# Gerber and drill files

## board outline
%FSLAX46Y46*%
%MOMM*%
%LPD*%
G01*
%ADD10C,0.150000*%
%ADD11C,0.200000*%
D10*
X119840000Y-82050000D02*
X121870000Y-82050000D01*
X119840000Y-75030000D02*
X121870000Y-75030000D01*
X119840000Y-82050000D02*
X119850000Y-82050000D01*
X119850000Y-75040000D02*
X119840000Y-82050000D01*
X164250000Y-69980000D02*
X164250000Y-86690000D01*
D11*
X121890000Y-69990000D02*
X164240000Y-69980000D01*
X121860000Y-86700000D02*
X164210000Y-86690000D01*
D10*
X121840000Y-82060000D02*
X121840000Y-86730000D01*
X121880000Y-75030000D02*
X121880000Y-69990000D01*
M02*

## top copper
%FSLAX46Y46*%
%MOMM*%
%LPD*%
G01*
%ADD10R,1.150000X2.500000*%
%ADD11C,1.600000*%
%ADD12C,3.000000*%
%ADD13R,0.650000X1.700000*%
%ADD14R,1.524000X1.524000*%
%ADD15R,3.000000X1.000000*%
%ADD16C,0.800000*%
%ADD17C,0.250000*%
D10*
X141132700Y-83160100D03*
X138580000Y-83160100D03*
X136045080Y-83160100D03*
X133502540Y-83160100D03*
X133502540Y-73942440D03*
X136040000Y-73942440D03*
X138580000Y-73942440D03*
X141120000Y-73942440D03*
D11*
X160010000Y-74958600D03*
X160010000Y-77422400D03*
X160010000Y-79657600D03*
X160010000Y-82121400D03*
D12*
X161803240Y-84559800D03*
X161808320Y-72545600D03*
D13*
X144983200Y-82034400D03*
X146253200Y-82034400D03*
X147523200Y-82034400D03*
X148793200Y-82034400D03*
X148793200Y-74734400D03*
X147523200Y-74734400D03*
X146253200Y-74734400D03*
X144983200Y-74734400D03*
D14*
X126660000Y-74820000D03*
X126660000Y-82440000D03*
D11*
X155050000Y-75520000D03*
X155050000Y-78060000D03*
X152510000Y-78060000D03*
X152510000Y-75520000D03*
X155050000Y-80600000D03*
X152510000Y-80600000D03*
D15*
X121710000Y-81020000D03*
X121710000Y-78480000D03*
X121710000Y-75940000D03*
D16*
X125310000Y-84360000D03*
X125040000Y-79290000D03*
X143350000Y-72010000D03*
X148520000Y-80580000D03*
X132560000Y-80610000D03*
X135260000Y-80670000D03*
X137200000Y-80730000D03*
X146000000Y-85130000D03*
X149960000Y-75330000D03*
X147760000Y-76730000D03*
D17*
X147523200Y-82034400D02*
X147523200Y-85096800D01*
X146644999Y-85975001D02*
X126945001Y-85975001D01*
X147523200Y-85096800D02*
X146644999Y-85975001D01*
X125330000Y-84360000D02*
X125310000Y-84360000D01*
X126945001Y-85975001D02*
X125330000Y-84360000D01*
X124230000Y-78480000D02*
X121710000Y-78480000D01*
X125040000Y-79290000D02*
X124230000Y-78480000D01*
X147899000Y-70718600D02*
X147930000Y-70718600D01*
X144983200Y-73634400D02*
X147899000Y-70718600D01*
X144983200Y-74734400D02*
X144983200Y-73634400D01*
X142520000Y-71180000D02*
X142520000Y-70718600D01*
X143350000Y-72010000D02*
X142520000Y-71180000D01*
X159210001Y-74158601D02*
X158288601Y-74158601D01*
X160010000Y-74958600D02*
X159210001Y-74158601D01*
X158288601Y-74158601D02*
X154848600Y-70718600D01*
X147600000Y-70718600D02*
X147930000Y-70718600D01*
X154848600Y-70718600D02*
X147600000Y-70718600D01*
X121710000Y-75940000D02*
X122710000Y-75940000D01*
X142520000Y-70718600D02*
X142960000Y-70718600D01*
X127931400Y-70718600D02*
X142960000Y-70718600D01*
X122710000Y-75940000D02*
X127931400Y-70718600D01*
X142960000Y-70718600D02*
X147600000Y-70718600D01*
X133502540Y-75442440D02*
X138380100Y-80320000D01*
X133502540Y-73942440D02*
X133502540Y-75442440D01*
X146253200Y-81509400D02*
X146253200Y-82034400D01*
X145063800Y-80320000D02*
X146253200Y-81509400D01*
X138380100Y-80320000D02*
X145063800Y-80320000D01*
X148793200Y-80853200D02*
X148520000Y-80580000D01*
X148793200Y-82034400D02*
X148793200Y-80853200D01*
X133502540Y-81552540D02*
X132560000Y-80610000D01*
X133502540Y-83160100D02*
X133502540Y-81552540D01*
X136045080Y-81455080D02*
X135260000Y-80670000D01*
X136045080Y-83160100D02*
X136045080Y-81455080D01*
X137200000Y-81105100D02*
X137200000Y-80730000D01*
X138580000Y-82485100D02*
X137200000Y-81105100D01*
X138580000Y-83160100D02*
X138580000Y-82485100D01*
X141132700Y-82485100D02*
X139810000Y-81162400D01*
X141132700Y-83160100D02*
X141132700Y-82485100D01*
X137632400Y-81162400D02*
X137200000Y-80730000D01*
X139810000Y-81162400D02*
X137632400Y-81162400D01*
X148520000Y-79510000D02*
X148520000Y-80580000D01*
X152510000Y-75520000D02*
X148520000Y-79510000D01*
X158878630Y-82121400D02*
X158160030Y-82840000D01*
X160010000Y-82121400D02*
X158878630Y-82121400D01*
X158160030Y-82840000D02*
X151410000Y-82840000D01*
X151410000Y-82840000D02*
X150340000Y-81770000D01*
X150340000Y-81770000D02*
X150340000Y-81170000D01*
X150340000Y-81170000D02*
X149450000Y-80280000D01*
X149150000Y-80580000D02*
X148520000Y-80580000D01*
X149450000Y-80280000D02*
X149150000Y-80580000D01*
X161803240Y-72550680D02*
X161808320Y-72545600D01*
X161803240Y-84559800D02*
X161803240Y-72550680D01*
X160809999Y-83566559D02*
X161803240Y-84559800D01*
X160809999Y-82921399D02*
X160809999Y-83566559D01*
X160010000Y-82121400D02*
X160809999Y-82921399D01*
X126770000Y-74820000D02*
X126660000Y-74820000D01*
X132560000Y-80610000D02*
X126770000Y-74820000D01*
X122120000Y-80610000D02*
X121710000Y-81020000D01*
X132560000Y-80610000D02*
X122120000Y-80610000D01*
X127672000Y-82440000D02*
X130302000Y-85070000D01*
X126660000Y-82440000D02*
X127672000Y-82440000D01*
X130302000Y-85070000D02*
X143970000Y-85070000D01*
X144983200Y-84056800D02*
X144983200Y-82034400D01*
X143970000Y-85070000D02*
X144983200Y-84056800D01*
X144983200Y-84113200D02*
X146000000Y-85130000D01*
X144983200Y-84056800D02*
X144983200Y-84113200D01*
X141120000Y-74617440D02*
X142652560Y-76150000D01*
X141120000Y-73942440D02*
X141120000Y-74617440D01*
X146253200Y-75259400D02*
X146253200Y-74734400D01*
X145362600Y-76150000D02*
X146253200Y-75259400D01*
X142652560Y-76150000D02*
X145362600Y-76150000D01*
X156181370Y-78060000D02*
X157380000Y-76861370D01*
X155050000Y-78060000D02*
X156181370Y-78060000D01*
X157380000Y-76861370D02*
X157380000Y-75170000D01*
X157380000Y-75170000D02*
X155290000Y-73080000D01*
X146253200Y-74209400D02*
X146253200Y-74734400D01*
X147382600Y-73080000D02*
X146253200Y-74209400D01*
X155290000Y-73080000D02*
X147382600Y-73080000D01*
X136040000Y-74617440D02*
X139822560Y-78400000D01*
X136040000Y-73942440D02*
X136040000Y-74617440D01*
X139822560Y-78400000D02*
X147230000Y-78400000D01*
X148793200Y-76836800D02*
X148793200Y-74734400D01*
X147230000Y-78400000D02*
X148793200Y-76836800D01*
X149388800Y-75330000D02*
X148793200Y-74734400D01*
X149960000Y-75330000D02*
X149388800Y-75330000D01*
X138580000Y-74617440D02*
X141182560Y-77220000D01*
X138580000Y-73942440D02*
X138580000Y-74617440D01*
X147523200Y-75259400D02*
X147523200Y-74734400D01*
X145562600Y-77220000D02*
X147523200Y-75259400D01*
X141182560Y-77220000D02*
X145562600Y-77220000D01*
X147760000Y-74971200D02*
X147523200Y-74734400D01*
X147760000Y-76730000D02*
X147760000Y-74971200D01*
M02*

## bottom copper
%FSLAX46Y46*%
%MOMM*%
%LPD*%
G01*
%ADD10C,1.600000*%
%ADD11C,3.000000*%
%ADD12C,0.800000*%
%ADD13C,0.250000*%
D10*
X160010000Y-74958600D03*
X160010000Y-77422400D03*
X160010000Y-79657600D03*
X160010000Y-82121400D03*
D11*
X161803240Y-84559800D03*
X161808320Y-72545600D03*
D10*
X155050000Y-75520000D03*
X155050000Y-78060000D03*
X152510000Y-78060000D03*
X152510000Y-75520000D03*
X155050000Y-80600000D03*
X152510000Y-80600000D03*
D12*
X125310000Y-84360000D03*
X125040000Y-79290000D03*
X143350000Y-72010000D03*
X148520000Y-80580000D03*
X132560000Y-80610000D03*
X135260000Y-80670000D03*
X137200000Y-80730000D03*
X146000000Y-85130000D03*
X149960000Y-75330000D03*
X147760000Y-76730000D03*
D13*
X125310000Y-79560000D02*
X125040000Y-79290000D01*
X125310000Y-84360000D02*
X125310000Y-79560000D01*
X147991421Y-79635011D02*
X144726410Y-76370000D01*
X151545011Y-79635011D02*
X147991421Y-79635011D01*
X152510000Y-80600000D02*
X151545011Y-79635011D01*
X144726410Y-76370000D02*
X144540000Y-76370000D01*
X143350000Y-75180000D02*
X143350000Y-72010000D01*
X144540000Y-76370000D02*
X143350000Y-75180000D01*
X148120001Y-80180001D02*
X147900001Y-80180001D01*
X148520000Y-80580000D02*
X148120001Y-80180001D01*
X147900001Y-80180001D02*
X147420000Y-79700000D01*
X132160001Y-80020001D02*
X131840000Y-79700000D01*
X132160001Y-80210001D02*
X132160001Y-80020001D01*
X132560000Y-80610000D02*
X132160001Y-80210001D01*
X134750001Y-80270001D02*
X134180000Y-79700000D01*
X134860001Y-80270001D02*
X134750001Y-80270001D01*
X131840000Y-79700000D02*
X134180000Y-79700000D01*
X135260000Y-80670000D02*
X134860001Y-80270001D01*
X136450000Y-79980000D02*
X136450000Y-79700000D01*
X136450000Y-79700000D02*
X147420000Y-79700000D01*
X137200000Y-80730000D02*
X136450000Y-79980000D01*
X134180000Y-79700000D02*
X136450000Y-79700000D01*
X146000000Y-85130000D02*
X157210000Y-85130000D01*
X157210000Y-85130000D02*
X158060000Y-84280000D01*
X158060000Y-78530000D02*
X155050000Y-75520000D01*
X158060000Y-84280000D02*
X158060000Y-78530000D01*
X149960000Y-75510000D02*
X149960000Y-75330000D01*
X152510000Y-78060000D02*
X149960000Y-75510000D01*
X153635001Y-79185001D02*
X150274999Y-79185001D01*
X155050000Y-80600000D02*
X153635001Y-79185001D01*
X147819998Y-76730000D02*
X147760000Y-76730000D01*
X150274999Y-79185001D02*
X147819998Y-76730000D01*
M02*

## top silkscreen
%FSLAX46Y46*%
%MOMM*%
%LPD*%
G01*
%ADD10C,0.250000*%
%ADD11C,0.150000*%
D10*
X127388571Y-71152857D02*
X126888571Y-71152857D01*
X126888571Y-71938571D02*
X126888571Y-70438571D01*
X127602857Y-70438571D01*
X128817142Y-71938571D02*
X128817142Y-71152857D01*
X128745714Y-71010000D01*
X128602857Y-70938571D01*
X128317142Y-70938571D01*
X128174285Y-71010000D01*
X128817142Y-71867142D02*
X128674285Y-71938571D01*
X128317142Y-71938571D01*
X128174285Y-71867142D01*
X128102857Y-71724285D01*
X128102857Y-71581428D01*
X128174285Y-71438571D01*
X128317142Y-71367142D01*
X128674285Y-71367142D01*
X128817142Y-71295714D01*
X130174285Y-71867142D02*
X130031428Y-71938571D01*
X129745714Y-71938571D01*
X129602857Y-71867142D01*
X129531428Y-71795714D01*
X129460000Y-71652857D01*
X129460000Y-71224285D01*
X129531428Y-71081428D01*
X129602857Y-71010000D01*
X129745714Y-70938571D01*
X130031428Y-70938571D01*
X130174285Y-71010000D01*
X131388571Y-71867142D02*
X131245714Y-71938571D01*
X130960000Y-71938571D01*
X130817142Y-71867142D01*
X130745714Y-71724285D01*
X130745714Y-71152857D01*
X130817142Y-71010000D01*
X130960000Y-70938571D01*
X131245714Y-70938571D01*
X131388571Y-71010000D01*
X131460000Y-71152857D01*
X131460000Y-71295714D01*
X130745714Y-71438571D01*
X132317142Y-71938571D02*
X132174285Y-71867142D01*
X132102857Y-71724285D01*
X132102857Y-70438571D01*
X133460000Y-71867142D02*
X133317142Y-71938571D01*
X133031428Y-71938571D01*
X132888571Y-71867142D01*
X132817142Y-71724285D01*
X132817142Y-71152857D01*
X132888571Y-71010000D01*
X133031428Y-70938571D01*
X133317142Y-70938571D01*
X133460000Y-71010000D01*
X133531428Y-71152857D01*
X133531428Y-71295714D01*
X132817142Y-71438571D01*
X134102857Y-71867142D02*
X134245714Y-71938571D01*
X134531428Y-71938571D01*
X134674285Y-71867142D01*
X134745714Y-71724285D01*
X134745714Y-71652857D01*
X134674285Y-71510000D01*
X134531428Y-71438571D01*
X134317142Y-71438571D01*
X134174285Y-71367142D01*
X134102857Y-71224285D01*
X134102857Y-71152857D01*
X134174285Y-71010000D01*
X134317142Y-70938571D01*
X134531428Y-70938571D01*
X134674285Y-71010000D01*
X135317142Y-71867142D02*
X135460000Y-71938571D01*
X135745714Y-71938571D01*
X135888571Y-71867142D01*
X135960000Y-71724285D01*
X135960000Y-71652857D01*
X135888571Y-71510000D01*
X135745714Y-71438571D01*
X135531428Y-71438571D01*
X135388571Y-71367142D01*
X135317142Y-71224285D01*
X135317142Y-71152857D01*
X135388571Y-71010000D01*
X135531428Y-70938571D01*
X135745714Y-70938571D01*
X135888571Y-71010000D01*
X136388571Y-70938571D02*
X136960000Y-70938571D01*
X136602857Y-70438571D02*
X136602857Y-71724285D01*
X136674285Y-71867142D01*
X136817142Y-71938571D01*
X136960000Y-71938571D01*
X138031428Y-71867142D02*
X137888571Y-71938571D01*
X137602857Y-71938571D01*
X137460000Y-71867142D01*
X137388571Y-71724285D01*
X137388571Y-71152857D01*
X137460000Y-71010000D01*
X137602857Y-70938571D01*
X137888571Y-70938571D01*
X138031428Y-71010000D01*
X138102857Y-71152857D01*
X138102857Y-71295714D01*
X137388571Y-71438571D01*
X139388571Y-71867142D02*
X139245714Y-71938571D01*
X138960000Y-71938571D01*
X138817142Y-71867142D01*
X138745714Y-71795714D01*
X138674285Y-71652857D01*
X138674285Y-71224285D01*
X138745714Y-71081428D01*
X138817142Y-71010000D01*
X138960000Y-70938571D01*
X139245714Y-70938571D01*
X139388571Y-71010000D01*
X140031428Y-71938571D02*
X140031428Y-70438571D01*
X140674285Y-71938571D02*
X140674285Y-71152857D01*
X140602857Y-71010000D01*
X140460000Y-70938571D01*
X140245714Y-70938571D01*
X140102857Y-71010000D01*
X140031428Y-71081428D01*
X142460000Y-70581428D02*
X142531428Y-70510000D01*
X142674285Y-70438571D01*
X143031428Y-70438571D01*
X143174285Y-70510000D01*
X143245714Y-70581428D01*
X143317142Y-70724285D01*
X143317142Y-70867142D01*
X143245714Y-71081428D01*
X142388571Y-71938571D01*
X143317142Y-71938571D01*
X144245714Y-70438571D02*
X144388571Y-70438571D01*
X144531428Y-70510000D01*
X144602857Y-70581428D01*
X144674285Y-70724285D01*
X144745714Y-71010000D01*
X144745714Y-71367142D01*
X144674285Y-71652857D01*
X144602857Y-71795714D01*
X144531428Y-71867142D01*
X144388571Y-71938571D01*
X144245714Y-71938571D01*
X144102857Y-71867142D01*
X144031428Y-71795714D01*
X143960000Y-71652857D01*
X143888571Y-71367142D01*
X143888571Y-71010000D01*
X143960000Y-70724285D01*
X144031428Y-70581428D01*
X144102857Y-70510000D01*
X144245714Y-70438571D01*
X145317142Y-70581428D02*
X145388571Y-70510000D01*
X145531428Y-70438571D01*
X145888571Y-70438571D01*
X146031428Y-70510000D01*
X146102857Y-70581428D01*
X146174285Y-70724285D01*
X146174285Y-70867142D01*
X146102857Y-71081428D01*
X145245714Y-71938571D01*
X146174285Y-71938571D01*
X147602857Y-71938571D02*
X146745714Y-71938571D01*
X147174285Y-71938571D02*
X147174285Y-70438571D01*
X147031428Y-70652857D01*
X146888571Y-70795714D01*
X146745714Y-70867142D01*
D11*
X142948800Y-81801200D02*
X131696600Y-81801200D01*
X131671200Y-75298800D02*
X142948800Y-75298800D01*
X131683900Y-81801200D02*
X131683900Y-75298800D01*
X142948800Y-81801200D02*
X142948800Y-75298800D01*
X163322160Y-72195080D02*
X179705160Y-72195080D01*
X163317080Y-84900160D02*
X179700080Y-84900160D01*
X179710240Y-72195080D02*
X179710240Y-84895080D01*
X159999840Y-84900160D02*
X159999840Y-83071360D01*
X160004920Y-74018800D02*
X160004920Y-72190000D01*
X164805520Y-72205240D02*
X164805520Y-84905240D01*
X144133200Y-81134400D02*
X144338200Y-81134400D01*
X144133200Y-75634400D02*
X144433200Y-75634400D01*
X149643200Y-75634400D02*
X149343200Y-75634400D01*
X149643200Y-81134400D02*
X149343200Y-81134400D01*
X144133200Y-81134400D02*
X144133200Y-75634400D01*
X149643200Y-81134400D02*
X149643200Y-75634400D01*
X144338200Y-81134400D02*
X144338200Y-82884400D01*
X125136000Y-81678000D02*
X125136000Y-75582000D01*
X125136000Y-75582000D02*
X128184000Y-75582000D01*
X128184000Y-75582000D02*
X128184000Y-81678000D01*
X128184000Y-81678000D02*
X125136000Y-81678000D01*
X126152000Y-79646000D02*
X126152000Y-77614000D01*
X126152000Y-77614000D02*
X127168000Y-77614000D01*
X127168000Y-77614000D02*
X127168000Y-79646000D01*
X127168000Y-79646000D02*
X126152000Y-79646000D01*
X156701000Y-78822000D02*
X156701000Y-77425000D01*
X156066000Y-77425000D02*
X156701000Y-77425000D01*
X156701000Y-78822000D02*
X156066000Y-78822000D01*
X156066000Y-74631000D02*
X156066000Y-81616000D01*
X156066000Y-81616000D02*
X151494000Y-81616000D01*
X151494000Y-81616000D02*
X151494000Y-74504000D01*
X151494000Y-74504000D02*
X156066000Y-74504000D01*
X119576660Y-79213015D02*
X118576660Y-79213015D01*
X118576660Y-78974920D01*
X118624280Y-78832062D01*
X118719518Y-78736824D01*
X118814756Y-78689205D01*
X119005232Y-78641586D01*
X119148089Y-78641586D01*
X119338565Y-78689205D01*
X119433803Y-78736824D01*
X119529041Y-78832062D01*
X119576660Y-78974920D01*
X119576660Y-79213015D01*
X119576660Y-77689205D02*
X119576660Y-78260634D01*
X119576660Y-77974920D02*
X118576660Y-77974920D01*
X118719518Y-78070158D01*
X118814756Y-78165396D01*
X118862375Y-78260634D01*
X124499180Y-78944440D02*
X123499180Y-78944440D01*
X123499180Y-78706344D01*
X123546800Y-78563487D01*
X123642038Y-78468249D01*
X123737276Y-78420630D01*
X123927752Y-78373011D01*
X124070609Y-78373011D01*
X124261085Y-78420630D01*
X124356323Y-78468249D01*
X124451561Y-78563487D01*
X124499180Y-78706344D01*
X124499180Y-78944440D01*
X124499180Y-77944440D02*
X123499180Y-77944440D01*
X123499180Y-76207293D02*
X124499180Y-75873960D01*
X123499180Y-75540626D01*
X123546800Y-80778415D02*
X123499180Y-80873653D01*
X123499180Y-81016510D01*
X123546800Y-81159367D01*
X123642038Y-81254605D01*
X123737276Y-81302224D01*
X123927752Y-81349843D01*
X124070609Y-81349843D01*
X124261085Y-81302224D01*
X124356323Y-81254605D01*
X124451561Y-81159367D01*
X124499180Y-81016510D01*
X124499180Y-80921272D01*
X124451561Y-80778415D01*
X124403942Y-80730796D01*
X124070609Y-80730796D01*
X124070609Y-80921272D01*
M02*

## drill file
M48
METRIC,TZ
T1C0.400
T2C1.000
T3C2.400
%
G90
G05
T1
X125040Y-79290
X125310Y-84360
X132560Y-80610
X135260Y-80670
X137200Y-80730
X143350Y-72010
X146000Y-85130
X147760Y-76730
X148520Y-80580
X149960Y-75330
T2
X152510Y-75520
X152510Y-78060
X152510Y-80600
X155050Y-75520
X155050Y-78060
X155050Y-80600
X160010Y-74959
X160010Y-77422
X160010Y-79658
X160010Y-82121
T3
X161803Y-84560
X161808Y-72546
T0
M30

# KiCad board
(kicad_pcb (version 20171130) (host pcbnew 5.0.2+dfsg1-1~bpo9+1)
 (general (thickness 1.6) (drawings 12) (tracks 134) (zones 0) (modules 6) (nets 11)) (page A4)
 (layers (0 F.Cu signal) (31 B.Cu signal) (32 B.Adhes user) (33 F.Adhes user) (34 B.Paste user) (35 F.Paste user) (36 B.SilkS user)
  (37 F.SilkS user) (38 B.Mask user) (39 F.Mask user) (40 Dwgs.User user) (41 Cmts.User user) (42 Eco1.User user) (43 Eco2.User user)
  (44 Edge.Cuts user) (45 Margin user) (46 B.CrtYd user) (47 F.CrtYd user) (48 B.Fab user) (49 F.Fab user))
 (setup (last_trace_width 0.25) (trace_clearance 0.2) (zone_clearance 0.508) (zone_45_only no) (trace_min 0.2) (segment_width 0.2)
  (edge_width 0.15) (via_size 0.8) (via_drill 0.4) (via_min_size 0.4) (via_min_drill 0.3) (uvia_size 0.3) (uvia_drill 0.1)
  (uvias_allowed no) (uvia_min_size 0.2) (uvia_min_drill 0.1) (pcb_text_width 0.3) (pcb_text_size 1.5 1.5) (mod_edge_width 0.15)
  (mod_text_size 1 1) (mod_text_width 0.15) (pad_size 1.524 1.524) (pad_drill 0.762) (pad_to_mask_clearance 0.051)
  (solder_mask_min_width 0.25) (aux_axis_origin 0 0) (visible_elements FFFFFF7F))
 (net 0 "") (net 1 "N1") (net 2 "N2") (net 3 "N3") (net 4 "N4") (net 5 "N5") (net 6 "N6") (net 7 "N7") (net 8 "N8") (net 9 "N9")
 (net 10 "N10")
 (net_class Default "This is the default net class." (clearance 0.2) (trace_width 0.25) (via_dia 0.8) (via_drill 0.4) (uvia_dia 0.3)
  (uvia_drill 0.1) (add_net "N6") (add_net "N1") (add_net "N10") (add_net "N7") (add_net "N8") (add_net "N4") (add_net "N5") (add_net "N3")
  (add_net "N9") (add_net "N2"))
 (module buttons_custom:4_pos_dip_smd (layer F.Cu) (at 137.31 78.55 180)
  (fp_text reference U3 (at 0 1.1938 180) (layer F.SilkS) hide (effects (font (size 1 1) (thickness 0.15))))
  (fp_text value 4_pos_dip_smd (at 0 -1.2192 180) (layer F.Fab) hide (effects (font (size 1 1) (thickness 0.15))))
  (fp_line (start -5.6388 -3.2512) (end 5.6134 -3.2512) (layer F.SilkS) (width 0.15))
  (fp_line (start 5.6388 3.2512) (end -5.6388 3.2512) (layer F.SilkS) (width 0.15))
  (fp_line (start 5.6261 -3.2512) (end 5.6261 3.2512) (layer F.SilkS) (width 0.15))
  (fp_line (start -5.6388 -3.2512) (end -5.6388 3.2512) (layer F.SilkS) (width 0.15))
  (pad 1 smd rect (at -3.8227 -4.6101 180) (size 1.15 2.5) (layers F.Cu F.Paste F.Mask) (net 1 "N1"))
  (pad 2 smd rect (at -1.27 -4.6101 180) (size 1.15 2.5) (layers F.Cu F.Paste F.Mask) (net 1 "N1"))
  (pad 3 smd rect (at 1.26492 -4.6101 180) (size 1.15 2.5) (layers F.Cu F.Paste F.Mask) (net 1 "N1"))
  (pad 4 smd rect (at 3.80746 -4.6101 180) (size 1.15 2.5) (layers F.Cu F.Paste F.Mask) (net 1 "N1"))
  (pad 5 smd rect (at 3.80746 4.60756 180) (size 1.15 2.5) (layers F.Cu F.Paste F.Mask) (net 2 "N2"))
  (pad 6 smd rect (at 1.27 4.60756 180) (size 1.15 2.5) (layers F.Cu F.Paste F.Mask) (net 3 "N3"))
  (pad 7 smd rect (at -1.27 4.60756 180) (size 1.15 2.5) (layers F.Cu F.Paste F.Mask) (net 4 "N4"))
  (pad 8 smd rect (at -3.81 4.60756 180) (size 1.15 2.5) (layers F.Cu F.Paste F.Mask) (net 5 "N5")))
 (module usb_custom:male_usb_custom (layer F.Cu) (at 160.01 78.54 270)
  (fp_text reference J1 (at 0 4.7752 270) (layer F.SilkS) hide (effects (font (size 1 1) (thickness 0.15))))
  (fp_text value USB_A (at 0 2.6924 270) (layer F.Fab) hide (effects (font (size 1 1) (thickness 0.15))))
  (fp_line (start -6.34492 -3.31216) (end -6.34492 -19.69516) (layer F.SilkS) (width 0.15))
  (fp_line (start 6.36016 -3.30708) (end 6.36016 -19.69008) (layer F.SilkS) (width 0.15))
  (fp_line (start -6.34492 -19.70024) (end 6.35508 -19.70024) (layer F.SilkS) (width 0.15))
  (fp_line (start 6.36016 0.01016) (end 4.53136 0.01016) (layer F.SilkS) (width 0.15))
  (fp_line (start -4.5212 0.00508) (end -6.35 0.00508) (layer F.SilkS) (width 0.15))
  (fp_line (start -6.33476 -4.79552) (end 6.36524 -4.79552) (layer F.SilkS) (width 0.15))
  (pad 1 thru_hole circle (at -3.5814 0 270) (size 1.6 1.6) (drill 1) (layers *.Cu *.Mask) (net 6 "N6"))
  (pad 2 thru_hole circle (at -1.1176 0 270) (size 1.6 1.6) (drill 1) (layers *.Cu *.Mask) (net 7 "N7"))
  (pad 3 thru_hole circle (at 1.1176 0 270) (size 1.6 1.6) (drill 1) (layers *.Cu *.Mask) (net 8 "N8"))
  (pad 4 thru_hole circle (at 3.5814 0 270) (size 1.6 1.6) (drill 1) (layers *.Cu *.Mask) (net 1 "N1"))
  (pad 4 thru_hole circle (at 6.0198 -1.79324 270) (size 3 3) (drill 2.4) (layers *.Cu *.Mask) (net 1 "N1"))
  (pad 4 thru_hole circle (at -5.9944 -1.79832 270) (size 3 3) (drill 2.4) (layers *.Cu *.Mask) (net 1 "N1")))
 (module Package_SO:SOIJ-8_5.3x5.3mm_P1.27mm (layer F.Cu) (at 146.8882 78.3844 90)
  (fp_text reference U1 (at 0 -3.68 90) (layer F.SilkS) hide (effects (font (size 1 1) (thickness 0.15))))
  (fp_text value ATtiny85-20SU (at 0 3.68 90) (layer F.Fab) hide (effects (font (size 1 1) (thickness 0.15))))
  (fp_line (start -2.75 -2.755) (end -2.75 -2.55) (layer F.SilkS) (width 0.15))
  (fp_line (start 2.75 -2.755) (end 2.75 -2.455) (layer F.SilkS) (width 0.15))
  (fp_line (start 2.75 2.755) (end 2.75 2.455) (layer F.SilkS) (width 0.15))
  (fp_line (start -2.75 2.755) (end -2.75 2.455) (layer F.SilkS) (width 0.15))
  (fp_line (start -2.75 -2.755) (end 2.75 -2.755) (layer F.SilkS) (width 0.15))
  (fp_line (start -2.75 2.755) (end 2.75 2.755) (layer F.SilkS) (width 0.15))
  (fp_line (start -2.75 -2.55) (end -4.5 -2.55) (layer F.SilkS) (width 0.15))
  (pad 1 smd rect (at -3.65 -1.905 90) (size 1.7 0.65) (layers F.Cu F.Paste F.Mask) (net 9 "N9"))
  (pad 2 smd rect (at -3.65 -0.635 90) (size 1.7 0.65) (layers F.Cu F.Paste F.Mask) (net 2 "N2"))
  (pad 3 smd rect (at -3.65 0.635 90) (size 1.7 0.65) (layers F.Cu F.Paste F.Mask) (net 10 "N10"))
  (pad 4 smd rect (at -3.65 1.905 90) (size 1.7 0.65) (layers F.Cu F.Paste F.Mask) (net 1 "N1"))
  (pad 5 smd rect (at 3.65 1.905 90) (size 1.7 0.65) (layers F.Cu F.Paste F.Mask) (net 3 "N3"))
  (pad 6 smd rect (at 3.65 0.635 90) (size 1.7 0.65) (layers F.Cu F.Paste F.Mask) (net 4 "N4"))
  (pad 7 smd rect (at 3.65 -0.635 90) (size 1.7 0.65) (layers F.Cu F.Paste F.Mask) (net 5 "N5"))
  (pad 8 smd rect (at 3.65 -1.905 90) (size 1.7 0.65) (layers F.Cu F.Paste F.Mask) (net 6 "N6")))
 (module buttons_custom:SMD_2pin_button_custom (layer F.Cu) (at 126.66 78.63 90)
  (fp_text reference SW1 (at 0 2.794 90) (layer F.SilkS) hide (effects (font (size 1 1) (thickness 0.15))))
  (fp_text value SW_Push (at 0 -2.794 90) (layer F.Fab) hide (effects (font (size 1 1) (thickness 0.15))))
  (fp_line (start -3.048 -1.524) (end 3.048 -1.524) (layer F.SilkS) (width 0.15))
  (fp_line (start 3.048 -1.524) (end 3.048 1.524) (layer F.SilkS) (width 0.15))
  (fp_line (start 3.048 1.524) (end -3.048 1.524) (layer F.SilkS) (width 0.15))
  (fp_line (start -3.048 1.524) (end -3.048 -1.524) (layer F.SilkS) (width 0.15))
  (fp_line (start -1.016 -0.508) (end 1.016 -0.508) (layer F.SilkS) (width 0.15))
  (fp_line (start 1.016 -0.508) (end 1.016 0.508) (layer F.SilkS) (width 0.15))
  (fp_line (start 1.016 0.508) (end -1.016 0.508) (layer F.SilkS) (width 0.15))
  (fp_line (start -1.016 0.508) (end -1.016 -0.508) (layer F.SilkS) (width 0.15))
  (pad 1 smd rect (at 3.81 0 90) (size 1.524 1.524) (layers F.Cu F.Paste F.Mask) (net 1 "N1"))
  (pad 2 smd rect (at -3.81 0 90) (size 1.524 1.524) (layers F.Cu F.Paste F.Mask) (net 9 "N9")))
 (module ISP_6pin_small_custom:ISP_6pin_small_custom (layer F.Cu) (at 153.78 78.06 270)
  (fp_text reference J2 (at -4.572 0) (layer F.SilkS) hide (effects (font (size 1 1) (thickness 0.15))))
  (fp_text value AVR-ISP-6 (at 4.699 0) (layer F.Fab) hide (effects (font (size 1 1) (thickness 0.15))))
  (fp_line (start 0.762 -2.921) (end -0.635 -2.921) (layer F.SilkS) (width 0.15))
  (fp_line (start -0.635 -2.286) (end -0.635 -2.921) (layer F.SilkS) (width 0.15))
  (fp_line (start 0.762 -2.921) (end 0.762 -2.286) (layer F.SilkS) (width 0.15))
  (fp_line (start -3.429 -2.286) (end 3.556 -2.286) (layer F.SilkS) (width 0.15))
  (fp_line (start 3.556 -2.286) (end 3.556 2.286) (layer F.SilkS) (width 0.15))
  (fp_line (start 3.556 2.286) (end -3.556 2.286) (layer F.SilkS) (width 0.15))
  (fp_line (start -3.556 2.286) (end -3.556 -2.286) (layer F.SilkS) (width 0.15))
  (pad 5 thru_hole circle (at -2.54 -1.27 270) (size 1.6 1.6) (drill 1) (layers *.Cu *.Mask) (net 9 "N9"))
  (pad 3 thru_hole circle (at 0 -1.27 270) (size 1.6 1.6) (drill 1) (layers *.Cu *.Mask) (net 5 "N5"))
  (pad 4 thru_hole circle (at 0 1.27 270) (size 1.6 1.6) (drill 1) (layers *.Cu *.Mask) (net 3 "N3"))
  (pad 6 thru_hole circle (at -2.54 1.27 270) (size 1.6 1.6) (drill 1) (layers *.Cu *.Mask) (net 1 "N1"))
  (pad 1 thru_hole circle (at 2.54 -1.27 270) (size 1.6 1.6) (drill 1) (layers *.Cu *.Mask) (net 4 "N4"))
  (pad 2 thru_hole circle (at 2.54 1.27 270) (size 1.6 1.6) (drill 1) (layers *.Cu *.Mask) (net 6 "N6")))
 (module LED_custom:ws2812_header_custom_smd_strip (layer F.Cu) (at 121.71 78.48 90)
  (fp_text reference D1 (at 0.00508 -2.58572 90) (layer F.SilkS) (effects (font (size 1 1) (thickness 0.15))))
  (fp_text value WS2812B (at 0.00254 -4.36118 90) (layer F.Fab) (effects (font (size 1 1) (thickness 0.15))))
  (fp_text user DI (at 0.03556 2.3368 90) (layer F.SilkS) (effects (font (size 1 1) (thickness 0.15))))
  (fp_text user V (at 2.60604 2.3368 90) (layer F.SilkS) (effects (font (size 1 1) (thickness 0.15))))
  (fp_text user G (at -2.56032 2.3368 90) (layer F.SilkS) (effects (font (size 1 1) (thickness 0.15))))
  (pad 3 smd rect (at -2.54 0 90) (size 1 3) (layers F.Cu F.Paste F.Mask) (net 1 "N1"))
  (pad 4 smd rect (at 0 0 90) (size 1 3) (layers F.Cu F.Paste F.Mask) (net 10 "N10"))
  (pad 1 smd rect (at 2.54 0 90) (size 1 3) (layers F.Cu F.Paste F.Mask) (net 6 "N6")))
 (gr_line (start 119.84 82.05) (end 121.87 82.05) (layer Edge.Cuts) (width 0.15))
 (gr_line (start 119.84 75.03) (end 121.87 75.03) (layer Edge.Cuts) (width 0.15))
 (gr_line (start 119.84 82.05) (end 119.85 82.05) (layer Edge.Cuts) (width 0.15))
 (gr_line (start 119.85 75.04) (end 119.84 82.05) (layer Edge.Cuts) (width 0.15))
 (gr_line (start 164.25 69.98) (end 164.25 86.69) (layer Edge.Cuts) (width 0.15))
 (gr_line (start 121.89 69.99) (end 164.24 69.98) (layer Edge.Cuts) (width 0.2))
 (gr_line (start 121.86 86.7) (end 164.21 86.69) (layer Edge.Cuts) (width 0.2))
 (gr_line (start 121.84 82.06) (end 121.84 86.73) (layer Edge.Cuts) (width 0.15))
 (gr_line (start 121.88 75.03) (end 121.88 69.99) (layer Edge.Cuts) (width 0.15))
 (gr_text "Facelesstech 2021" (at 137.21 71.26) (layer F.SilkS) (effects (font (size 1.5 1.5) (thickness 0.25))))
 (segment (start 147.5232 82.0344) (end 147.5232 85.0968) (width 0.25) (layer F.Cu) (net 10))
 (segment (start 146.644999 85.975001) (end 126.945001 85.975001) (width 0.25) (layer F.Cu) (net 10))
 (segment (start 147.5232 85.0968) (end 146.644999 85.975001) (width 0.25) (layer F.Cu) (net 10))
 (via (at 125.31 84.36) (size 0.8) (drill 0.4) (layers F.Cu B.Cu) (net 10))
 (segment (start 125.33 84.36) (end 125.31 84.36) (width 0.25) (layer F.Cu) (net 10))
 (segment (start 126.945001 85.975001) (end 125.33 84.36) (width 0.25) (layer F.Cu) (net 10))
 (via (at 125.04 79.29) (size 0.8) (drill 0.4) (layers F.Cu B.Cu) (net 10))
 (segment (start 125.31 79.56) (end 125.04 79.29) (width 0.25) (layer B.Cu) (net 10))
 (segment (start 125.31 84.36) (end 125.31 79.56) (width 0.25) (layer B.Cu) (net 10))
 (segment (start 124.23 78.48) (end 121.71 78.48) (width 0.25) (layer F.Cu) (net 10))
 (segment (start 125.04 79.29) (end 124.23 78.48) (width 0.25) (layer F.Cu) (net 10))
 (segment (start 147.899 70.7186) (end 147.93 70.7186) (width 0.25) (layer F.Cu) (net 6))
 (segment (start 144.9832 73.6344) (end 147.899 70.7186) (width 0.25) (layer F.Cu) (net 6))
 (segment (start 144.9832 74.7344) (end 144.9832 73.6344) (width 0.25) (layer F.Cu) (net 6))
 (segment (start 147.991421 79.635011) (end 144.72641 76.37) (width 0.25) (layer B.Cu) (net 6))
 (segment (start 151.545011 79.635011) (end 147.991421 79.635011) (width 0.25) (layer B.Cu) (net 6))
 (segment (start 152.51 80.6) (end 151.545011 79.635011) (width 0.25) (layer B.Cu) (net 6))
 (segment (start 144.72641 76.37) (end 144.54 76.37) (width 0.25) (layer B.Cu) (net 6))
 (segment (start 143.35 75.18) (end 143.35 72.01) (width 0.25) (layer B.Cu) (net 6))
 (via (at 143.35 72.01) (size 0.8) (drill 0.4) (layers F.Cu B.Cu) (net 6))
 (segment (start 144.54 76.37) (end 143.35 75.18) (width 0.25) (layer B.Cu) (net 6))
 (segment (start 142.52 71.18) (end 142.52 70.7186) (width 0.25) (layer F.Cu) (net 6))
 (segment (start 143.35 72.01) (end 142.52 71.18) (width 0.25) (layer F.Cu) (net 6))
 (segment (start 159.210001 74.158601) (end 158.288601 74.158601) (width 0.25) (layer F.Cu) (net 6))
 (segment (start 160.01 74.9586) (end 159.210001 74.158601) (width 0.25) (layer F.Cu) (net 6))
 (segment (start 158.288601 74.158601) (end 154.8486 70.7186) (width 0.25) (layer F.Cu) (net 6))
 (segment (start 147.6 70.7186) (end 147.93 70.7186) (width 0.25) (layer F.Cu) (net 6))
 (segment (start 154.8486 70.7186) (end 147.6 70.7186) (width 0.25) (layer F.Cu) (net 6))
 (segment (start 121.71 75.94) (end 122.71 75.94) (width 0.25) (layer F.Cu) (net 6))
 (segment (start 142.52 70.7186) (end 142.96 70.7186) (width 0.25) (layer F.Cu) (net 6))
 (segment (start 127.9314 70.7186) (end 142.96 70.7186) (width 0.25) (layer F.Cu) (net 6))
 (segment (start 122.71 75.94) (end 127.9314 70.7186) (width 0.25) (layer F.Cu) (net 6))
 (segment (start 142.96 70.7186) (end 147.6 70.7186) (width 0.25) (layer F.Cu) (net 6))
 (segment (start 133.50254 75.44244) (end 138.3801 80.32) (width 0.25) (layer F.Cu) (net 2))
 (segment (start 133.50254 73.94244) (end 133.50254 75.44244) (width 0.25) (layer F.Cu) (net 2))
 (segment (start 146.2532 81.5094) (end 146.2532 82.0344) (width 0.25) (layer F.Cu) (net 2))
 (segment (start 145.0638 80.32) (end 146.2532 81.5094) (width 0.25) (layer F.Cu) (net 2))
 (segment (start 138.3801 80.32) (end 145.0638 80.32) (width 0.25) (layer F.Cu) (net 2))
 (via (at 148.52 80.58) (size 0.8) (drill 0.4) (layers F.Cu B.Cu) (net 1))
 (segment (start 148.7932 80.8532) (end 148.52 80.58) (width 0.25) (layer F.Cu) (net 1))
 (segment (start 148.7932 82.0344) (end 148.7932 80.8532) (width 0.25) (layer F.Cu) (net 1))
 (segment (start 148.120001 80.180001) (end 147.900001 80.180001) (width 0.25) (layer B.Cu) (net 1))
 (segment (start 148.52 80.58) (end 148.120001 80.180001) (width 0.25) (layer B.Cu) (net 1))
 (segment (start 147.900001 80.180001) (end 147.42 79.7) (width 0.25) (layer B.Cu) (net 1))
 (via (at 132.56 80.61) (size 0.8) (drill 0.4) (layers F.Cu B.Cu) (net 1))
 (segment (start 133.50254 81.55254) (end 132.56 80.61) (width 0.25) (layer F.Cu) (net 1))
 (segment (start 133.50254 83.1601) (end 133.50254 81.55254) (width 0.25) (layer F.Cu) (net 1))
 (segment (start 132.160001 80.020001) (end 131.84 79.7) (width 0.25) (layer B.Cu) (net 1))
 (segment (start 132.160001 80.210001) (end 132.160001 80.020001) (width 0.25) (layer B.Cu) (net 1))
 (segment (start 132.56 80.61) (end 132.160001 80.210001) (width 0.25) (layer B.Cu) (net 1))
 (segment (start 136.04508 81.45508) (end 135.26 80.67) (width 0.25) (layer F.Cu) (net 1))
 (via (at 135.26 80.67) (size 0.8) (drill 0.4) (layers F.Cu B.Cu) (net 1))
 (segment (start 136.04508 83.1601) (end 136.04508 81.45508) (width 0.25) (layer F.Cu) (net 1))
 (segment (start 134.750001 80.270001) (end 134.18 79.7) (width 0.25) (layer B.Cu) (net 1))
 (segment (start 134.860001 80.270001) (end 134.750001 80.270001) (width 0.25) (layer B.Cu) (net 1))
 (segment (start 131.84 79.7) (end 134.18 79.7) (width 0.25) (layer B.Cu) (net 1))
 (segment (start 135.26 80.67) (end 134.860001 80.270001) (width 0.25) (layer B.Cu) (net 1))
 (segment (start 137.2 81.1051) (end 137.2 80.73) (width 0.25) (layer F.Cu) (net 1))
 (via (at 137.2 80.73) (size 0.8) (drill 0.4) (layers F.Cu B.Cu) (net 1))
 (segment (start 138.58 82.4851) (end 137.2 81.1051) (width 0.25) (layer F.Cu) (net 1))
 (segment (start 138.58 83.1601) (end 138.58 82.4851) (width 0.25) (layer F.Cu) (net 1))
 (segment (start 136.45 79.98) (end 136.45 79.7) (width 0.25) (layer B.Cu) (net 1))
 (segment (start 136.45 79.7) (end 147.42 79.7) (width 0.25) (layer B.Cu) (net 1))
 (segment (start 137.2 80.73) (end 136.45 79.98) (width 0.25) (layer B.Cu) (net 1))
 (segment (start 134.18 79.7) (end 136.45 79.7) (width 0.25) (layer B.Cu) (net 1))
 (segment (start 141.1327 82.4851) (end 139.81 81.1624) (width 0.25) (layer F.Cu) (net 1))
 (segment (start 141.1327 83.1601) (end 141.1327 82.4851) (width 0.25) (layer F.Cu) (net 1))
 (segment (start 137.6324 81.1624) (end 137.2 80.73) (width 0.25) (layer F.Cu) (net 1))
 (segment (start 139.81 81.1624) (end 137.6324 81.1624) (width 0.25) (layer F.Cu) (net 1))
 (segment (start 148.52 79.51) (end 148.52 80.58) (width 0.25) (layer F.Cu) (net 1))
 (segment (start 152.51 75.52) (end 148.52 79.51) (width 0.25) (layer F.Cu) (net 1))
 (segment (start 158.87863 82.1214) (end 158.16003 82.84) (width 0.25) (layer F.Cu) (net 1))
 (segment (start 160.01 82.1214) (end 158.87863 82.1214) (width 0.25) (layer F.Cu) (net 1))
 (segment (start 158.16003 82.84) (end 151.41 82.84) (width 0.25) (layer F.Cu) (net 1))
 (segment (start 151.41 82.84) (end 150.34 81.77) (width 0.25) (layer F.Cu) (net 1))
 (segment (start 150.34 81.77) (end 150.34 81.17) (width 0.25) (layer F.Cu) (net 1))
 (segment (start 150.34 81.17) (end 149.45 80.28) (width 0.25) (layer F.Cu) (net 1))
 (segment (start 149.15 80.58) (end 148.52 80.58) (width 0.25) (layer F.Cu) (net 1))
 (segment (start 149.45 80.28) (end 149.15 80.58) (width 0.25) (layer F.Cu) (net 1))
 (segment (start 161.80324 72.55068) (end 161.80832 72.5456) (width 0.25) (layer F.Cu) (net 1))
 (segment (start 161.80324 84.5598) (end 161.80324 72.55068) (width 0.25) (layer F.Cu) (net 1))
 (segment (start 160.809999 83.566559) (end 161.80324 84.5598) (width 0.25) (layer F.Cu) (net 1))
 (segment (start 160.809999 82.921399) (end 160.809999 83.566559) (width 0.25) (layer F.Cu) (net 1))
 (segment (start 160.01 82.1214) (end 160.809999 82.921399) (width 0.25) (layer F.Cu) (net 1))
 (segment (start 126.77 74.82) (end 126.66 74.82) (width 0.25) (layer F.Cu) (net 1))
 (segment (start 132.56 80.61) (end 126.77 74.82) (width 0.25) (layer F.Cu) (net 1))
 (segment (start 122.12 80.61) (end 121.71 81.02) (width 0.25) (layer F.Cu) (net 1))
 (segment (start 132.56 80.61) (end 122.12 80.61) (width 0.25) (layer F.Cu) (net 1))
 (segment (start 127.672 82.44) (end 130.302 85.07) (width 0.25) (layer F.Cu) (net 9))
 (segment (start 126.66 82.44) (end 127.672 82.44) (width 0.25) (layer F.Cu) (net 9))
 (segment (start 130.302 85.07) (end 143.97 85.07) (width 0.25) (layer F.Cu) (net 9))
 (segment (start 144.9832 84.0568) (end 144.9832 82.0344) (width 0.25) (layer F.Cu) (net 9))
 (segment (start 143.97 85.07) (end 144.9832 84.0568) (width 0.25) (layer F.Cu) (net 9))
 (via (at 146 85.13) (size 0.8) (drill 0.4) (layers F.Cu B.Cu) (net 9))
 (segment (start 144.9832 84.1132) (end 146 85.13) (width 0.25) (layer F.Cu) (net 9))
 (segment (start 144.9832 84.0568) (end 144.9832 84.1132) (width 0.25) (layer F.Cu) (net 9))
 (segment (start 146 85.13) (end 157.21 85.13) (width 0.25) (layer B.Cu) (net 9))
 (segment (start 157.21 85.13) (end 158.06 84.28) (width 0.25) (layer B.Cu) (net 9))
 (segment (start 158.06 78.53) (end 155.05 75.52) (width 0.25) (layer B.Cu) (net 9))
 (segment (start 158.06 84.28) (end 158.06 78.53) (width 0.25) (layer B.Cu) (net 9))
 (segment (start 141.12 74.61744) (end 142.65256 76.15) (width 0.25) (layer F.Cu) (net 5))
 (segment (start 141.12 73.94244) (end 141.12 74.61744) (width 0.25) (layer F.Cu) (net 5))
 (segment (start 146.2532 75.2594) (end 146.2532 74.7344) (width 0.25) (layer F.Cu) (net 5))
 (segment (start 145.3626 76.15) (end 146.2532 75.2594) (width 0.25) (layer F.Cu) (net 5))
 (segment (start 142.65256 76.15) (end 145.3626 76.15) (width 0.25) (layer F.Cu) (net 5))
 (segment (start 156.18137 78.06) (end 157.38 76.86137) (width 0.25) (layer F.Cu) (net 5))
 (segment (start 155.05 78.06) (end 156.18137 78.06) (width 0.25) (layer F.Cu) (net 5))
 (segment (start 157.38 76.86137) (end 157.38 75.17) (width 0.25) (layer F.Cu) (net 5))
 (segment (start 157.38 75.17) (end 155.29 73.08) (width 0.25) (layer F.Cu) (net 5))
 (segment (start 146.2532 74.2094) (end 146.2532 74.7344) (width 0.25) (layer F.Cu) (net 5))
 (segment (start 147.3826 73.08) (end 146.2532 74.2094) (width 0.25) (layer F.Cu) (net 5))
 (segment (start 155.29 73.08) (end 147.3826 73.08) (width 0.25) (layer F.Cu) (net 5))
 (segment (start 136.04 74.61744) (end 139.82256 78.4) (width 0.25) (layer F.Cu) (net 3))
 (segment (start 136.04 73.94244) (end 136.04 74.61744) (width 0.25) (layer F.Cu) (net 3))
 (segment (start 139.82256 78.4) (end 147.23 78.4) (width 0.25) (layer F.Cu) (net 3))
 (segment (start 148.7932 76.8368) (end 148.7932 74.7344) (width 0.25) (layer F.Cu) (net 3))
 (segment (start 147.23 78.4) (end 148.7932 76.8368) (width 0.25) (layer F.Cu) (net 3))
 (segment (start 149.96 75.51) (end 149.96 75.33) (width 0.25) (layer B.Cu) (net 3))
 (via (at 149.96 75.33) (size 0.8) (drill 0.4) (layers F.Cu B.Cu) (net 3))
 (segment (start 152.51 78.06) (end 149.96 75.51) (width 0.25) (layer B.Cu) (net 3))
 (segment (start 149.3888 75.33) (end 148.7932 74.7344) (width 0.25) (layer F.Cu) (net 3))
 (segment (start 149.96 75.33) (end 149.3888 75.33) (width 0.25) (layer F.Cu) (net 3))
 (segment (start 138.58 74.61744) (end 141.18256 77.22) (width 0.25) (layer F.Cu) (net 4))
 (segment (start 138.58 73.94244) (end 138.58 74.61744) (width 0.25) (layer F.Cu) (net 4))
 (segment (start 147.5232 75.2594) (end 147.5232 74.7344) (width 0.25) (layer F.Cu) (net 4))
 (segment (start 145.5626 77.22) (end 147.5232 75.2594) (width 0.25) (layer F.Cu) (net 4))
 (segment (start 141.18256 77.22) (end 145.5626 77.22) (width 0.25) (layer F.Cu) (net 4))
 (segment (start 153.635001 79.185001) (end 150.274999 79.185001) (width 0.25) (layer B.Cu) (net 4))
 (segment (start 155.05 80.6) (end 153.635001 79.185001) (width 0.25) (layer B.Cu) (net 4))
 (segment (start 147.819998 76.73) (end 147.76 76.73) (width 0.25) (layer B.Cu) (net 4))
 (via (at 147.76 76.73) (size 0.8) (drill 0.4) (layers F.Cu B.Cu) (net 4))
 (segment (start 150.274999 79.185001) (end 147.819998 76.73) (width 0.25) (layer B.Cu) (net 4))
 (segment (start 147.76 74.9712) (end 147.5232 74.7344) (width 0.25) (layer F.Cu) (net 4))
 (segment (start 147.76 76.73) (end 147.76 74.9712) (width 0.25) (layer F.Cu) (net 4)))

